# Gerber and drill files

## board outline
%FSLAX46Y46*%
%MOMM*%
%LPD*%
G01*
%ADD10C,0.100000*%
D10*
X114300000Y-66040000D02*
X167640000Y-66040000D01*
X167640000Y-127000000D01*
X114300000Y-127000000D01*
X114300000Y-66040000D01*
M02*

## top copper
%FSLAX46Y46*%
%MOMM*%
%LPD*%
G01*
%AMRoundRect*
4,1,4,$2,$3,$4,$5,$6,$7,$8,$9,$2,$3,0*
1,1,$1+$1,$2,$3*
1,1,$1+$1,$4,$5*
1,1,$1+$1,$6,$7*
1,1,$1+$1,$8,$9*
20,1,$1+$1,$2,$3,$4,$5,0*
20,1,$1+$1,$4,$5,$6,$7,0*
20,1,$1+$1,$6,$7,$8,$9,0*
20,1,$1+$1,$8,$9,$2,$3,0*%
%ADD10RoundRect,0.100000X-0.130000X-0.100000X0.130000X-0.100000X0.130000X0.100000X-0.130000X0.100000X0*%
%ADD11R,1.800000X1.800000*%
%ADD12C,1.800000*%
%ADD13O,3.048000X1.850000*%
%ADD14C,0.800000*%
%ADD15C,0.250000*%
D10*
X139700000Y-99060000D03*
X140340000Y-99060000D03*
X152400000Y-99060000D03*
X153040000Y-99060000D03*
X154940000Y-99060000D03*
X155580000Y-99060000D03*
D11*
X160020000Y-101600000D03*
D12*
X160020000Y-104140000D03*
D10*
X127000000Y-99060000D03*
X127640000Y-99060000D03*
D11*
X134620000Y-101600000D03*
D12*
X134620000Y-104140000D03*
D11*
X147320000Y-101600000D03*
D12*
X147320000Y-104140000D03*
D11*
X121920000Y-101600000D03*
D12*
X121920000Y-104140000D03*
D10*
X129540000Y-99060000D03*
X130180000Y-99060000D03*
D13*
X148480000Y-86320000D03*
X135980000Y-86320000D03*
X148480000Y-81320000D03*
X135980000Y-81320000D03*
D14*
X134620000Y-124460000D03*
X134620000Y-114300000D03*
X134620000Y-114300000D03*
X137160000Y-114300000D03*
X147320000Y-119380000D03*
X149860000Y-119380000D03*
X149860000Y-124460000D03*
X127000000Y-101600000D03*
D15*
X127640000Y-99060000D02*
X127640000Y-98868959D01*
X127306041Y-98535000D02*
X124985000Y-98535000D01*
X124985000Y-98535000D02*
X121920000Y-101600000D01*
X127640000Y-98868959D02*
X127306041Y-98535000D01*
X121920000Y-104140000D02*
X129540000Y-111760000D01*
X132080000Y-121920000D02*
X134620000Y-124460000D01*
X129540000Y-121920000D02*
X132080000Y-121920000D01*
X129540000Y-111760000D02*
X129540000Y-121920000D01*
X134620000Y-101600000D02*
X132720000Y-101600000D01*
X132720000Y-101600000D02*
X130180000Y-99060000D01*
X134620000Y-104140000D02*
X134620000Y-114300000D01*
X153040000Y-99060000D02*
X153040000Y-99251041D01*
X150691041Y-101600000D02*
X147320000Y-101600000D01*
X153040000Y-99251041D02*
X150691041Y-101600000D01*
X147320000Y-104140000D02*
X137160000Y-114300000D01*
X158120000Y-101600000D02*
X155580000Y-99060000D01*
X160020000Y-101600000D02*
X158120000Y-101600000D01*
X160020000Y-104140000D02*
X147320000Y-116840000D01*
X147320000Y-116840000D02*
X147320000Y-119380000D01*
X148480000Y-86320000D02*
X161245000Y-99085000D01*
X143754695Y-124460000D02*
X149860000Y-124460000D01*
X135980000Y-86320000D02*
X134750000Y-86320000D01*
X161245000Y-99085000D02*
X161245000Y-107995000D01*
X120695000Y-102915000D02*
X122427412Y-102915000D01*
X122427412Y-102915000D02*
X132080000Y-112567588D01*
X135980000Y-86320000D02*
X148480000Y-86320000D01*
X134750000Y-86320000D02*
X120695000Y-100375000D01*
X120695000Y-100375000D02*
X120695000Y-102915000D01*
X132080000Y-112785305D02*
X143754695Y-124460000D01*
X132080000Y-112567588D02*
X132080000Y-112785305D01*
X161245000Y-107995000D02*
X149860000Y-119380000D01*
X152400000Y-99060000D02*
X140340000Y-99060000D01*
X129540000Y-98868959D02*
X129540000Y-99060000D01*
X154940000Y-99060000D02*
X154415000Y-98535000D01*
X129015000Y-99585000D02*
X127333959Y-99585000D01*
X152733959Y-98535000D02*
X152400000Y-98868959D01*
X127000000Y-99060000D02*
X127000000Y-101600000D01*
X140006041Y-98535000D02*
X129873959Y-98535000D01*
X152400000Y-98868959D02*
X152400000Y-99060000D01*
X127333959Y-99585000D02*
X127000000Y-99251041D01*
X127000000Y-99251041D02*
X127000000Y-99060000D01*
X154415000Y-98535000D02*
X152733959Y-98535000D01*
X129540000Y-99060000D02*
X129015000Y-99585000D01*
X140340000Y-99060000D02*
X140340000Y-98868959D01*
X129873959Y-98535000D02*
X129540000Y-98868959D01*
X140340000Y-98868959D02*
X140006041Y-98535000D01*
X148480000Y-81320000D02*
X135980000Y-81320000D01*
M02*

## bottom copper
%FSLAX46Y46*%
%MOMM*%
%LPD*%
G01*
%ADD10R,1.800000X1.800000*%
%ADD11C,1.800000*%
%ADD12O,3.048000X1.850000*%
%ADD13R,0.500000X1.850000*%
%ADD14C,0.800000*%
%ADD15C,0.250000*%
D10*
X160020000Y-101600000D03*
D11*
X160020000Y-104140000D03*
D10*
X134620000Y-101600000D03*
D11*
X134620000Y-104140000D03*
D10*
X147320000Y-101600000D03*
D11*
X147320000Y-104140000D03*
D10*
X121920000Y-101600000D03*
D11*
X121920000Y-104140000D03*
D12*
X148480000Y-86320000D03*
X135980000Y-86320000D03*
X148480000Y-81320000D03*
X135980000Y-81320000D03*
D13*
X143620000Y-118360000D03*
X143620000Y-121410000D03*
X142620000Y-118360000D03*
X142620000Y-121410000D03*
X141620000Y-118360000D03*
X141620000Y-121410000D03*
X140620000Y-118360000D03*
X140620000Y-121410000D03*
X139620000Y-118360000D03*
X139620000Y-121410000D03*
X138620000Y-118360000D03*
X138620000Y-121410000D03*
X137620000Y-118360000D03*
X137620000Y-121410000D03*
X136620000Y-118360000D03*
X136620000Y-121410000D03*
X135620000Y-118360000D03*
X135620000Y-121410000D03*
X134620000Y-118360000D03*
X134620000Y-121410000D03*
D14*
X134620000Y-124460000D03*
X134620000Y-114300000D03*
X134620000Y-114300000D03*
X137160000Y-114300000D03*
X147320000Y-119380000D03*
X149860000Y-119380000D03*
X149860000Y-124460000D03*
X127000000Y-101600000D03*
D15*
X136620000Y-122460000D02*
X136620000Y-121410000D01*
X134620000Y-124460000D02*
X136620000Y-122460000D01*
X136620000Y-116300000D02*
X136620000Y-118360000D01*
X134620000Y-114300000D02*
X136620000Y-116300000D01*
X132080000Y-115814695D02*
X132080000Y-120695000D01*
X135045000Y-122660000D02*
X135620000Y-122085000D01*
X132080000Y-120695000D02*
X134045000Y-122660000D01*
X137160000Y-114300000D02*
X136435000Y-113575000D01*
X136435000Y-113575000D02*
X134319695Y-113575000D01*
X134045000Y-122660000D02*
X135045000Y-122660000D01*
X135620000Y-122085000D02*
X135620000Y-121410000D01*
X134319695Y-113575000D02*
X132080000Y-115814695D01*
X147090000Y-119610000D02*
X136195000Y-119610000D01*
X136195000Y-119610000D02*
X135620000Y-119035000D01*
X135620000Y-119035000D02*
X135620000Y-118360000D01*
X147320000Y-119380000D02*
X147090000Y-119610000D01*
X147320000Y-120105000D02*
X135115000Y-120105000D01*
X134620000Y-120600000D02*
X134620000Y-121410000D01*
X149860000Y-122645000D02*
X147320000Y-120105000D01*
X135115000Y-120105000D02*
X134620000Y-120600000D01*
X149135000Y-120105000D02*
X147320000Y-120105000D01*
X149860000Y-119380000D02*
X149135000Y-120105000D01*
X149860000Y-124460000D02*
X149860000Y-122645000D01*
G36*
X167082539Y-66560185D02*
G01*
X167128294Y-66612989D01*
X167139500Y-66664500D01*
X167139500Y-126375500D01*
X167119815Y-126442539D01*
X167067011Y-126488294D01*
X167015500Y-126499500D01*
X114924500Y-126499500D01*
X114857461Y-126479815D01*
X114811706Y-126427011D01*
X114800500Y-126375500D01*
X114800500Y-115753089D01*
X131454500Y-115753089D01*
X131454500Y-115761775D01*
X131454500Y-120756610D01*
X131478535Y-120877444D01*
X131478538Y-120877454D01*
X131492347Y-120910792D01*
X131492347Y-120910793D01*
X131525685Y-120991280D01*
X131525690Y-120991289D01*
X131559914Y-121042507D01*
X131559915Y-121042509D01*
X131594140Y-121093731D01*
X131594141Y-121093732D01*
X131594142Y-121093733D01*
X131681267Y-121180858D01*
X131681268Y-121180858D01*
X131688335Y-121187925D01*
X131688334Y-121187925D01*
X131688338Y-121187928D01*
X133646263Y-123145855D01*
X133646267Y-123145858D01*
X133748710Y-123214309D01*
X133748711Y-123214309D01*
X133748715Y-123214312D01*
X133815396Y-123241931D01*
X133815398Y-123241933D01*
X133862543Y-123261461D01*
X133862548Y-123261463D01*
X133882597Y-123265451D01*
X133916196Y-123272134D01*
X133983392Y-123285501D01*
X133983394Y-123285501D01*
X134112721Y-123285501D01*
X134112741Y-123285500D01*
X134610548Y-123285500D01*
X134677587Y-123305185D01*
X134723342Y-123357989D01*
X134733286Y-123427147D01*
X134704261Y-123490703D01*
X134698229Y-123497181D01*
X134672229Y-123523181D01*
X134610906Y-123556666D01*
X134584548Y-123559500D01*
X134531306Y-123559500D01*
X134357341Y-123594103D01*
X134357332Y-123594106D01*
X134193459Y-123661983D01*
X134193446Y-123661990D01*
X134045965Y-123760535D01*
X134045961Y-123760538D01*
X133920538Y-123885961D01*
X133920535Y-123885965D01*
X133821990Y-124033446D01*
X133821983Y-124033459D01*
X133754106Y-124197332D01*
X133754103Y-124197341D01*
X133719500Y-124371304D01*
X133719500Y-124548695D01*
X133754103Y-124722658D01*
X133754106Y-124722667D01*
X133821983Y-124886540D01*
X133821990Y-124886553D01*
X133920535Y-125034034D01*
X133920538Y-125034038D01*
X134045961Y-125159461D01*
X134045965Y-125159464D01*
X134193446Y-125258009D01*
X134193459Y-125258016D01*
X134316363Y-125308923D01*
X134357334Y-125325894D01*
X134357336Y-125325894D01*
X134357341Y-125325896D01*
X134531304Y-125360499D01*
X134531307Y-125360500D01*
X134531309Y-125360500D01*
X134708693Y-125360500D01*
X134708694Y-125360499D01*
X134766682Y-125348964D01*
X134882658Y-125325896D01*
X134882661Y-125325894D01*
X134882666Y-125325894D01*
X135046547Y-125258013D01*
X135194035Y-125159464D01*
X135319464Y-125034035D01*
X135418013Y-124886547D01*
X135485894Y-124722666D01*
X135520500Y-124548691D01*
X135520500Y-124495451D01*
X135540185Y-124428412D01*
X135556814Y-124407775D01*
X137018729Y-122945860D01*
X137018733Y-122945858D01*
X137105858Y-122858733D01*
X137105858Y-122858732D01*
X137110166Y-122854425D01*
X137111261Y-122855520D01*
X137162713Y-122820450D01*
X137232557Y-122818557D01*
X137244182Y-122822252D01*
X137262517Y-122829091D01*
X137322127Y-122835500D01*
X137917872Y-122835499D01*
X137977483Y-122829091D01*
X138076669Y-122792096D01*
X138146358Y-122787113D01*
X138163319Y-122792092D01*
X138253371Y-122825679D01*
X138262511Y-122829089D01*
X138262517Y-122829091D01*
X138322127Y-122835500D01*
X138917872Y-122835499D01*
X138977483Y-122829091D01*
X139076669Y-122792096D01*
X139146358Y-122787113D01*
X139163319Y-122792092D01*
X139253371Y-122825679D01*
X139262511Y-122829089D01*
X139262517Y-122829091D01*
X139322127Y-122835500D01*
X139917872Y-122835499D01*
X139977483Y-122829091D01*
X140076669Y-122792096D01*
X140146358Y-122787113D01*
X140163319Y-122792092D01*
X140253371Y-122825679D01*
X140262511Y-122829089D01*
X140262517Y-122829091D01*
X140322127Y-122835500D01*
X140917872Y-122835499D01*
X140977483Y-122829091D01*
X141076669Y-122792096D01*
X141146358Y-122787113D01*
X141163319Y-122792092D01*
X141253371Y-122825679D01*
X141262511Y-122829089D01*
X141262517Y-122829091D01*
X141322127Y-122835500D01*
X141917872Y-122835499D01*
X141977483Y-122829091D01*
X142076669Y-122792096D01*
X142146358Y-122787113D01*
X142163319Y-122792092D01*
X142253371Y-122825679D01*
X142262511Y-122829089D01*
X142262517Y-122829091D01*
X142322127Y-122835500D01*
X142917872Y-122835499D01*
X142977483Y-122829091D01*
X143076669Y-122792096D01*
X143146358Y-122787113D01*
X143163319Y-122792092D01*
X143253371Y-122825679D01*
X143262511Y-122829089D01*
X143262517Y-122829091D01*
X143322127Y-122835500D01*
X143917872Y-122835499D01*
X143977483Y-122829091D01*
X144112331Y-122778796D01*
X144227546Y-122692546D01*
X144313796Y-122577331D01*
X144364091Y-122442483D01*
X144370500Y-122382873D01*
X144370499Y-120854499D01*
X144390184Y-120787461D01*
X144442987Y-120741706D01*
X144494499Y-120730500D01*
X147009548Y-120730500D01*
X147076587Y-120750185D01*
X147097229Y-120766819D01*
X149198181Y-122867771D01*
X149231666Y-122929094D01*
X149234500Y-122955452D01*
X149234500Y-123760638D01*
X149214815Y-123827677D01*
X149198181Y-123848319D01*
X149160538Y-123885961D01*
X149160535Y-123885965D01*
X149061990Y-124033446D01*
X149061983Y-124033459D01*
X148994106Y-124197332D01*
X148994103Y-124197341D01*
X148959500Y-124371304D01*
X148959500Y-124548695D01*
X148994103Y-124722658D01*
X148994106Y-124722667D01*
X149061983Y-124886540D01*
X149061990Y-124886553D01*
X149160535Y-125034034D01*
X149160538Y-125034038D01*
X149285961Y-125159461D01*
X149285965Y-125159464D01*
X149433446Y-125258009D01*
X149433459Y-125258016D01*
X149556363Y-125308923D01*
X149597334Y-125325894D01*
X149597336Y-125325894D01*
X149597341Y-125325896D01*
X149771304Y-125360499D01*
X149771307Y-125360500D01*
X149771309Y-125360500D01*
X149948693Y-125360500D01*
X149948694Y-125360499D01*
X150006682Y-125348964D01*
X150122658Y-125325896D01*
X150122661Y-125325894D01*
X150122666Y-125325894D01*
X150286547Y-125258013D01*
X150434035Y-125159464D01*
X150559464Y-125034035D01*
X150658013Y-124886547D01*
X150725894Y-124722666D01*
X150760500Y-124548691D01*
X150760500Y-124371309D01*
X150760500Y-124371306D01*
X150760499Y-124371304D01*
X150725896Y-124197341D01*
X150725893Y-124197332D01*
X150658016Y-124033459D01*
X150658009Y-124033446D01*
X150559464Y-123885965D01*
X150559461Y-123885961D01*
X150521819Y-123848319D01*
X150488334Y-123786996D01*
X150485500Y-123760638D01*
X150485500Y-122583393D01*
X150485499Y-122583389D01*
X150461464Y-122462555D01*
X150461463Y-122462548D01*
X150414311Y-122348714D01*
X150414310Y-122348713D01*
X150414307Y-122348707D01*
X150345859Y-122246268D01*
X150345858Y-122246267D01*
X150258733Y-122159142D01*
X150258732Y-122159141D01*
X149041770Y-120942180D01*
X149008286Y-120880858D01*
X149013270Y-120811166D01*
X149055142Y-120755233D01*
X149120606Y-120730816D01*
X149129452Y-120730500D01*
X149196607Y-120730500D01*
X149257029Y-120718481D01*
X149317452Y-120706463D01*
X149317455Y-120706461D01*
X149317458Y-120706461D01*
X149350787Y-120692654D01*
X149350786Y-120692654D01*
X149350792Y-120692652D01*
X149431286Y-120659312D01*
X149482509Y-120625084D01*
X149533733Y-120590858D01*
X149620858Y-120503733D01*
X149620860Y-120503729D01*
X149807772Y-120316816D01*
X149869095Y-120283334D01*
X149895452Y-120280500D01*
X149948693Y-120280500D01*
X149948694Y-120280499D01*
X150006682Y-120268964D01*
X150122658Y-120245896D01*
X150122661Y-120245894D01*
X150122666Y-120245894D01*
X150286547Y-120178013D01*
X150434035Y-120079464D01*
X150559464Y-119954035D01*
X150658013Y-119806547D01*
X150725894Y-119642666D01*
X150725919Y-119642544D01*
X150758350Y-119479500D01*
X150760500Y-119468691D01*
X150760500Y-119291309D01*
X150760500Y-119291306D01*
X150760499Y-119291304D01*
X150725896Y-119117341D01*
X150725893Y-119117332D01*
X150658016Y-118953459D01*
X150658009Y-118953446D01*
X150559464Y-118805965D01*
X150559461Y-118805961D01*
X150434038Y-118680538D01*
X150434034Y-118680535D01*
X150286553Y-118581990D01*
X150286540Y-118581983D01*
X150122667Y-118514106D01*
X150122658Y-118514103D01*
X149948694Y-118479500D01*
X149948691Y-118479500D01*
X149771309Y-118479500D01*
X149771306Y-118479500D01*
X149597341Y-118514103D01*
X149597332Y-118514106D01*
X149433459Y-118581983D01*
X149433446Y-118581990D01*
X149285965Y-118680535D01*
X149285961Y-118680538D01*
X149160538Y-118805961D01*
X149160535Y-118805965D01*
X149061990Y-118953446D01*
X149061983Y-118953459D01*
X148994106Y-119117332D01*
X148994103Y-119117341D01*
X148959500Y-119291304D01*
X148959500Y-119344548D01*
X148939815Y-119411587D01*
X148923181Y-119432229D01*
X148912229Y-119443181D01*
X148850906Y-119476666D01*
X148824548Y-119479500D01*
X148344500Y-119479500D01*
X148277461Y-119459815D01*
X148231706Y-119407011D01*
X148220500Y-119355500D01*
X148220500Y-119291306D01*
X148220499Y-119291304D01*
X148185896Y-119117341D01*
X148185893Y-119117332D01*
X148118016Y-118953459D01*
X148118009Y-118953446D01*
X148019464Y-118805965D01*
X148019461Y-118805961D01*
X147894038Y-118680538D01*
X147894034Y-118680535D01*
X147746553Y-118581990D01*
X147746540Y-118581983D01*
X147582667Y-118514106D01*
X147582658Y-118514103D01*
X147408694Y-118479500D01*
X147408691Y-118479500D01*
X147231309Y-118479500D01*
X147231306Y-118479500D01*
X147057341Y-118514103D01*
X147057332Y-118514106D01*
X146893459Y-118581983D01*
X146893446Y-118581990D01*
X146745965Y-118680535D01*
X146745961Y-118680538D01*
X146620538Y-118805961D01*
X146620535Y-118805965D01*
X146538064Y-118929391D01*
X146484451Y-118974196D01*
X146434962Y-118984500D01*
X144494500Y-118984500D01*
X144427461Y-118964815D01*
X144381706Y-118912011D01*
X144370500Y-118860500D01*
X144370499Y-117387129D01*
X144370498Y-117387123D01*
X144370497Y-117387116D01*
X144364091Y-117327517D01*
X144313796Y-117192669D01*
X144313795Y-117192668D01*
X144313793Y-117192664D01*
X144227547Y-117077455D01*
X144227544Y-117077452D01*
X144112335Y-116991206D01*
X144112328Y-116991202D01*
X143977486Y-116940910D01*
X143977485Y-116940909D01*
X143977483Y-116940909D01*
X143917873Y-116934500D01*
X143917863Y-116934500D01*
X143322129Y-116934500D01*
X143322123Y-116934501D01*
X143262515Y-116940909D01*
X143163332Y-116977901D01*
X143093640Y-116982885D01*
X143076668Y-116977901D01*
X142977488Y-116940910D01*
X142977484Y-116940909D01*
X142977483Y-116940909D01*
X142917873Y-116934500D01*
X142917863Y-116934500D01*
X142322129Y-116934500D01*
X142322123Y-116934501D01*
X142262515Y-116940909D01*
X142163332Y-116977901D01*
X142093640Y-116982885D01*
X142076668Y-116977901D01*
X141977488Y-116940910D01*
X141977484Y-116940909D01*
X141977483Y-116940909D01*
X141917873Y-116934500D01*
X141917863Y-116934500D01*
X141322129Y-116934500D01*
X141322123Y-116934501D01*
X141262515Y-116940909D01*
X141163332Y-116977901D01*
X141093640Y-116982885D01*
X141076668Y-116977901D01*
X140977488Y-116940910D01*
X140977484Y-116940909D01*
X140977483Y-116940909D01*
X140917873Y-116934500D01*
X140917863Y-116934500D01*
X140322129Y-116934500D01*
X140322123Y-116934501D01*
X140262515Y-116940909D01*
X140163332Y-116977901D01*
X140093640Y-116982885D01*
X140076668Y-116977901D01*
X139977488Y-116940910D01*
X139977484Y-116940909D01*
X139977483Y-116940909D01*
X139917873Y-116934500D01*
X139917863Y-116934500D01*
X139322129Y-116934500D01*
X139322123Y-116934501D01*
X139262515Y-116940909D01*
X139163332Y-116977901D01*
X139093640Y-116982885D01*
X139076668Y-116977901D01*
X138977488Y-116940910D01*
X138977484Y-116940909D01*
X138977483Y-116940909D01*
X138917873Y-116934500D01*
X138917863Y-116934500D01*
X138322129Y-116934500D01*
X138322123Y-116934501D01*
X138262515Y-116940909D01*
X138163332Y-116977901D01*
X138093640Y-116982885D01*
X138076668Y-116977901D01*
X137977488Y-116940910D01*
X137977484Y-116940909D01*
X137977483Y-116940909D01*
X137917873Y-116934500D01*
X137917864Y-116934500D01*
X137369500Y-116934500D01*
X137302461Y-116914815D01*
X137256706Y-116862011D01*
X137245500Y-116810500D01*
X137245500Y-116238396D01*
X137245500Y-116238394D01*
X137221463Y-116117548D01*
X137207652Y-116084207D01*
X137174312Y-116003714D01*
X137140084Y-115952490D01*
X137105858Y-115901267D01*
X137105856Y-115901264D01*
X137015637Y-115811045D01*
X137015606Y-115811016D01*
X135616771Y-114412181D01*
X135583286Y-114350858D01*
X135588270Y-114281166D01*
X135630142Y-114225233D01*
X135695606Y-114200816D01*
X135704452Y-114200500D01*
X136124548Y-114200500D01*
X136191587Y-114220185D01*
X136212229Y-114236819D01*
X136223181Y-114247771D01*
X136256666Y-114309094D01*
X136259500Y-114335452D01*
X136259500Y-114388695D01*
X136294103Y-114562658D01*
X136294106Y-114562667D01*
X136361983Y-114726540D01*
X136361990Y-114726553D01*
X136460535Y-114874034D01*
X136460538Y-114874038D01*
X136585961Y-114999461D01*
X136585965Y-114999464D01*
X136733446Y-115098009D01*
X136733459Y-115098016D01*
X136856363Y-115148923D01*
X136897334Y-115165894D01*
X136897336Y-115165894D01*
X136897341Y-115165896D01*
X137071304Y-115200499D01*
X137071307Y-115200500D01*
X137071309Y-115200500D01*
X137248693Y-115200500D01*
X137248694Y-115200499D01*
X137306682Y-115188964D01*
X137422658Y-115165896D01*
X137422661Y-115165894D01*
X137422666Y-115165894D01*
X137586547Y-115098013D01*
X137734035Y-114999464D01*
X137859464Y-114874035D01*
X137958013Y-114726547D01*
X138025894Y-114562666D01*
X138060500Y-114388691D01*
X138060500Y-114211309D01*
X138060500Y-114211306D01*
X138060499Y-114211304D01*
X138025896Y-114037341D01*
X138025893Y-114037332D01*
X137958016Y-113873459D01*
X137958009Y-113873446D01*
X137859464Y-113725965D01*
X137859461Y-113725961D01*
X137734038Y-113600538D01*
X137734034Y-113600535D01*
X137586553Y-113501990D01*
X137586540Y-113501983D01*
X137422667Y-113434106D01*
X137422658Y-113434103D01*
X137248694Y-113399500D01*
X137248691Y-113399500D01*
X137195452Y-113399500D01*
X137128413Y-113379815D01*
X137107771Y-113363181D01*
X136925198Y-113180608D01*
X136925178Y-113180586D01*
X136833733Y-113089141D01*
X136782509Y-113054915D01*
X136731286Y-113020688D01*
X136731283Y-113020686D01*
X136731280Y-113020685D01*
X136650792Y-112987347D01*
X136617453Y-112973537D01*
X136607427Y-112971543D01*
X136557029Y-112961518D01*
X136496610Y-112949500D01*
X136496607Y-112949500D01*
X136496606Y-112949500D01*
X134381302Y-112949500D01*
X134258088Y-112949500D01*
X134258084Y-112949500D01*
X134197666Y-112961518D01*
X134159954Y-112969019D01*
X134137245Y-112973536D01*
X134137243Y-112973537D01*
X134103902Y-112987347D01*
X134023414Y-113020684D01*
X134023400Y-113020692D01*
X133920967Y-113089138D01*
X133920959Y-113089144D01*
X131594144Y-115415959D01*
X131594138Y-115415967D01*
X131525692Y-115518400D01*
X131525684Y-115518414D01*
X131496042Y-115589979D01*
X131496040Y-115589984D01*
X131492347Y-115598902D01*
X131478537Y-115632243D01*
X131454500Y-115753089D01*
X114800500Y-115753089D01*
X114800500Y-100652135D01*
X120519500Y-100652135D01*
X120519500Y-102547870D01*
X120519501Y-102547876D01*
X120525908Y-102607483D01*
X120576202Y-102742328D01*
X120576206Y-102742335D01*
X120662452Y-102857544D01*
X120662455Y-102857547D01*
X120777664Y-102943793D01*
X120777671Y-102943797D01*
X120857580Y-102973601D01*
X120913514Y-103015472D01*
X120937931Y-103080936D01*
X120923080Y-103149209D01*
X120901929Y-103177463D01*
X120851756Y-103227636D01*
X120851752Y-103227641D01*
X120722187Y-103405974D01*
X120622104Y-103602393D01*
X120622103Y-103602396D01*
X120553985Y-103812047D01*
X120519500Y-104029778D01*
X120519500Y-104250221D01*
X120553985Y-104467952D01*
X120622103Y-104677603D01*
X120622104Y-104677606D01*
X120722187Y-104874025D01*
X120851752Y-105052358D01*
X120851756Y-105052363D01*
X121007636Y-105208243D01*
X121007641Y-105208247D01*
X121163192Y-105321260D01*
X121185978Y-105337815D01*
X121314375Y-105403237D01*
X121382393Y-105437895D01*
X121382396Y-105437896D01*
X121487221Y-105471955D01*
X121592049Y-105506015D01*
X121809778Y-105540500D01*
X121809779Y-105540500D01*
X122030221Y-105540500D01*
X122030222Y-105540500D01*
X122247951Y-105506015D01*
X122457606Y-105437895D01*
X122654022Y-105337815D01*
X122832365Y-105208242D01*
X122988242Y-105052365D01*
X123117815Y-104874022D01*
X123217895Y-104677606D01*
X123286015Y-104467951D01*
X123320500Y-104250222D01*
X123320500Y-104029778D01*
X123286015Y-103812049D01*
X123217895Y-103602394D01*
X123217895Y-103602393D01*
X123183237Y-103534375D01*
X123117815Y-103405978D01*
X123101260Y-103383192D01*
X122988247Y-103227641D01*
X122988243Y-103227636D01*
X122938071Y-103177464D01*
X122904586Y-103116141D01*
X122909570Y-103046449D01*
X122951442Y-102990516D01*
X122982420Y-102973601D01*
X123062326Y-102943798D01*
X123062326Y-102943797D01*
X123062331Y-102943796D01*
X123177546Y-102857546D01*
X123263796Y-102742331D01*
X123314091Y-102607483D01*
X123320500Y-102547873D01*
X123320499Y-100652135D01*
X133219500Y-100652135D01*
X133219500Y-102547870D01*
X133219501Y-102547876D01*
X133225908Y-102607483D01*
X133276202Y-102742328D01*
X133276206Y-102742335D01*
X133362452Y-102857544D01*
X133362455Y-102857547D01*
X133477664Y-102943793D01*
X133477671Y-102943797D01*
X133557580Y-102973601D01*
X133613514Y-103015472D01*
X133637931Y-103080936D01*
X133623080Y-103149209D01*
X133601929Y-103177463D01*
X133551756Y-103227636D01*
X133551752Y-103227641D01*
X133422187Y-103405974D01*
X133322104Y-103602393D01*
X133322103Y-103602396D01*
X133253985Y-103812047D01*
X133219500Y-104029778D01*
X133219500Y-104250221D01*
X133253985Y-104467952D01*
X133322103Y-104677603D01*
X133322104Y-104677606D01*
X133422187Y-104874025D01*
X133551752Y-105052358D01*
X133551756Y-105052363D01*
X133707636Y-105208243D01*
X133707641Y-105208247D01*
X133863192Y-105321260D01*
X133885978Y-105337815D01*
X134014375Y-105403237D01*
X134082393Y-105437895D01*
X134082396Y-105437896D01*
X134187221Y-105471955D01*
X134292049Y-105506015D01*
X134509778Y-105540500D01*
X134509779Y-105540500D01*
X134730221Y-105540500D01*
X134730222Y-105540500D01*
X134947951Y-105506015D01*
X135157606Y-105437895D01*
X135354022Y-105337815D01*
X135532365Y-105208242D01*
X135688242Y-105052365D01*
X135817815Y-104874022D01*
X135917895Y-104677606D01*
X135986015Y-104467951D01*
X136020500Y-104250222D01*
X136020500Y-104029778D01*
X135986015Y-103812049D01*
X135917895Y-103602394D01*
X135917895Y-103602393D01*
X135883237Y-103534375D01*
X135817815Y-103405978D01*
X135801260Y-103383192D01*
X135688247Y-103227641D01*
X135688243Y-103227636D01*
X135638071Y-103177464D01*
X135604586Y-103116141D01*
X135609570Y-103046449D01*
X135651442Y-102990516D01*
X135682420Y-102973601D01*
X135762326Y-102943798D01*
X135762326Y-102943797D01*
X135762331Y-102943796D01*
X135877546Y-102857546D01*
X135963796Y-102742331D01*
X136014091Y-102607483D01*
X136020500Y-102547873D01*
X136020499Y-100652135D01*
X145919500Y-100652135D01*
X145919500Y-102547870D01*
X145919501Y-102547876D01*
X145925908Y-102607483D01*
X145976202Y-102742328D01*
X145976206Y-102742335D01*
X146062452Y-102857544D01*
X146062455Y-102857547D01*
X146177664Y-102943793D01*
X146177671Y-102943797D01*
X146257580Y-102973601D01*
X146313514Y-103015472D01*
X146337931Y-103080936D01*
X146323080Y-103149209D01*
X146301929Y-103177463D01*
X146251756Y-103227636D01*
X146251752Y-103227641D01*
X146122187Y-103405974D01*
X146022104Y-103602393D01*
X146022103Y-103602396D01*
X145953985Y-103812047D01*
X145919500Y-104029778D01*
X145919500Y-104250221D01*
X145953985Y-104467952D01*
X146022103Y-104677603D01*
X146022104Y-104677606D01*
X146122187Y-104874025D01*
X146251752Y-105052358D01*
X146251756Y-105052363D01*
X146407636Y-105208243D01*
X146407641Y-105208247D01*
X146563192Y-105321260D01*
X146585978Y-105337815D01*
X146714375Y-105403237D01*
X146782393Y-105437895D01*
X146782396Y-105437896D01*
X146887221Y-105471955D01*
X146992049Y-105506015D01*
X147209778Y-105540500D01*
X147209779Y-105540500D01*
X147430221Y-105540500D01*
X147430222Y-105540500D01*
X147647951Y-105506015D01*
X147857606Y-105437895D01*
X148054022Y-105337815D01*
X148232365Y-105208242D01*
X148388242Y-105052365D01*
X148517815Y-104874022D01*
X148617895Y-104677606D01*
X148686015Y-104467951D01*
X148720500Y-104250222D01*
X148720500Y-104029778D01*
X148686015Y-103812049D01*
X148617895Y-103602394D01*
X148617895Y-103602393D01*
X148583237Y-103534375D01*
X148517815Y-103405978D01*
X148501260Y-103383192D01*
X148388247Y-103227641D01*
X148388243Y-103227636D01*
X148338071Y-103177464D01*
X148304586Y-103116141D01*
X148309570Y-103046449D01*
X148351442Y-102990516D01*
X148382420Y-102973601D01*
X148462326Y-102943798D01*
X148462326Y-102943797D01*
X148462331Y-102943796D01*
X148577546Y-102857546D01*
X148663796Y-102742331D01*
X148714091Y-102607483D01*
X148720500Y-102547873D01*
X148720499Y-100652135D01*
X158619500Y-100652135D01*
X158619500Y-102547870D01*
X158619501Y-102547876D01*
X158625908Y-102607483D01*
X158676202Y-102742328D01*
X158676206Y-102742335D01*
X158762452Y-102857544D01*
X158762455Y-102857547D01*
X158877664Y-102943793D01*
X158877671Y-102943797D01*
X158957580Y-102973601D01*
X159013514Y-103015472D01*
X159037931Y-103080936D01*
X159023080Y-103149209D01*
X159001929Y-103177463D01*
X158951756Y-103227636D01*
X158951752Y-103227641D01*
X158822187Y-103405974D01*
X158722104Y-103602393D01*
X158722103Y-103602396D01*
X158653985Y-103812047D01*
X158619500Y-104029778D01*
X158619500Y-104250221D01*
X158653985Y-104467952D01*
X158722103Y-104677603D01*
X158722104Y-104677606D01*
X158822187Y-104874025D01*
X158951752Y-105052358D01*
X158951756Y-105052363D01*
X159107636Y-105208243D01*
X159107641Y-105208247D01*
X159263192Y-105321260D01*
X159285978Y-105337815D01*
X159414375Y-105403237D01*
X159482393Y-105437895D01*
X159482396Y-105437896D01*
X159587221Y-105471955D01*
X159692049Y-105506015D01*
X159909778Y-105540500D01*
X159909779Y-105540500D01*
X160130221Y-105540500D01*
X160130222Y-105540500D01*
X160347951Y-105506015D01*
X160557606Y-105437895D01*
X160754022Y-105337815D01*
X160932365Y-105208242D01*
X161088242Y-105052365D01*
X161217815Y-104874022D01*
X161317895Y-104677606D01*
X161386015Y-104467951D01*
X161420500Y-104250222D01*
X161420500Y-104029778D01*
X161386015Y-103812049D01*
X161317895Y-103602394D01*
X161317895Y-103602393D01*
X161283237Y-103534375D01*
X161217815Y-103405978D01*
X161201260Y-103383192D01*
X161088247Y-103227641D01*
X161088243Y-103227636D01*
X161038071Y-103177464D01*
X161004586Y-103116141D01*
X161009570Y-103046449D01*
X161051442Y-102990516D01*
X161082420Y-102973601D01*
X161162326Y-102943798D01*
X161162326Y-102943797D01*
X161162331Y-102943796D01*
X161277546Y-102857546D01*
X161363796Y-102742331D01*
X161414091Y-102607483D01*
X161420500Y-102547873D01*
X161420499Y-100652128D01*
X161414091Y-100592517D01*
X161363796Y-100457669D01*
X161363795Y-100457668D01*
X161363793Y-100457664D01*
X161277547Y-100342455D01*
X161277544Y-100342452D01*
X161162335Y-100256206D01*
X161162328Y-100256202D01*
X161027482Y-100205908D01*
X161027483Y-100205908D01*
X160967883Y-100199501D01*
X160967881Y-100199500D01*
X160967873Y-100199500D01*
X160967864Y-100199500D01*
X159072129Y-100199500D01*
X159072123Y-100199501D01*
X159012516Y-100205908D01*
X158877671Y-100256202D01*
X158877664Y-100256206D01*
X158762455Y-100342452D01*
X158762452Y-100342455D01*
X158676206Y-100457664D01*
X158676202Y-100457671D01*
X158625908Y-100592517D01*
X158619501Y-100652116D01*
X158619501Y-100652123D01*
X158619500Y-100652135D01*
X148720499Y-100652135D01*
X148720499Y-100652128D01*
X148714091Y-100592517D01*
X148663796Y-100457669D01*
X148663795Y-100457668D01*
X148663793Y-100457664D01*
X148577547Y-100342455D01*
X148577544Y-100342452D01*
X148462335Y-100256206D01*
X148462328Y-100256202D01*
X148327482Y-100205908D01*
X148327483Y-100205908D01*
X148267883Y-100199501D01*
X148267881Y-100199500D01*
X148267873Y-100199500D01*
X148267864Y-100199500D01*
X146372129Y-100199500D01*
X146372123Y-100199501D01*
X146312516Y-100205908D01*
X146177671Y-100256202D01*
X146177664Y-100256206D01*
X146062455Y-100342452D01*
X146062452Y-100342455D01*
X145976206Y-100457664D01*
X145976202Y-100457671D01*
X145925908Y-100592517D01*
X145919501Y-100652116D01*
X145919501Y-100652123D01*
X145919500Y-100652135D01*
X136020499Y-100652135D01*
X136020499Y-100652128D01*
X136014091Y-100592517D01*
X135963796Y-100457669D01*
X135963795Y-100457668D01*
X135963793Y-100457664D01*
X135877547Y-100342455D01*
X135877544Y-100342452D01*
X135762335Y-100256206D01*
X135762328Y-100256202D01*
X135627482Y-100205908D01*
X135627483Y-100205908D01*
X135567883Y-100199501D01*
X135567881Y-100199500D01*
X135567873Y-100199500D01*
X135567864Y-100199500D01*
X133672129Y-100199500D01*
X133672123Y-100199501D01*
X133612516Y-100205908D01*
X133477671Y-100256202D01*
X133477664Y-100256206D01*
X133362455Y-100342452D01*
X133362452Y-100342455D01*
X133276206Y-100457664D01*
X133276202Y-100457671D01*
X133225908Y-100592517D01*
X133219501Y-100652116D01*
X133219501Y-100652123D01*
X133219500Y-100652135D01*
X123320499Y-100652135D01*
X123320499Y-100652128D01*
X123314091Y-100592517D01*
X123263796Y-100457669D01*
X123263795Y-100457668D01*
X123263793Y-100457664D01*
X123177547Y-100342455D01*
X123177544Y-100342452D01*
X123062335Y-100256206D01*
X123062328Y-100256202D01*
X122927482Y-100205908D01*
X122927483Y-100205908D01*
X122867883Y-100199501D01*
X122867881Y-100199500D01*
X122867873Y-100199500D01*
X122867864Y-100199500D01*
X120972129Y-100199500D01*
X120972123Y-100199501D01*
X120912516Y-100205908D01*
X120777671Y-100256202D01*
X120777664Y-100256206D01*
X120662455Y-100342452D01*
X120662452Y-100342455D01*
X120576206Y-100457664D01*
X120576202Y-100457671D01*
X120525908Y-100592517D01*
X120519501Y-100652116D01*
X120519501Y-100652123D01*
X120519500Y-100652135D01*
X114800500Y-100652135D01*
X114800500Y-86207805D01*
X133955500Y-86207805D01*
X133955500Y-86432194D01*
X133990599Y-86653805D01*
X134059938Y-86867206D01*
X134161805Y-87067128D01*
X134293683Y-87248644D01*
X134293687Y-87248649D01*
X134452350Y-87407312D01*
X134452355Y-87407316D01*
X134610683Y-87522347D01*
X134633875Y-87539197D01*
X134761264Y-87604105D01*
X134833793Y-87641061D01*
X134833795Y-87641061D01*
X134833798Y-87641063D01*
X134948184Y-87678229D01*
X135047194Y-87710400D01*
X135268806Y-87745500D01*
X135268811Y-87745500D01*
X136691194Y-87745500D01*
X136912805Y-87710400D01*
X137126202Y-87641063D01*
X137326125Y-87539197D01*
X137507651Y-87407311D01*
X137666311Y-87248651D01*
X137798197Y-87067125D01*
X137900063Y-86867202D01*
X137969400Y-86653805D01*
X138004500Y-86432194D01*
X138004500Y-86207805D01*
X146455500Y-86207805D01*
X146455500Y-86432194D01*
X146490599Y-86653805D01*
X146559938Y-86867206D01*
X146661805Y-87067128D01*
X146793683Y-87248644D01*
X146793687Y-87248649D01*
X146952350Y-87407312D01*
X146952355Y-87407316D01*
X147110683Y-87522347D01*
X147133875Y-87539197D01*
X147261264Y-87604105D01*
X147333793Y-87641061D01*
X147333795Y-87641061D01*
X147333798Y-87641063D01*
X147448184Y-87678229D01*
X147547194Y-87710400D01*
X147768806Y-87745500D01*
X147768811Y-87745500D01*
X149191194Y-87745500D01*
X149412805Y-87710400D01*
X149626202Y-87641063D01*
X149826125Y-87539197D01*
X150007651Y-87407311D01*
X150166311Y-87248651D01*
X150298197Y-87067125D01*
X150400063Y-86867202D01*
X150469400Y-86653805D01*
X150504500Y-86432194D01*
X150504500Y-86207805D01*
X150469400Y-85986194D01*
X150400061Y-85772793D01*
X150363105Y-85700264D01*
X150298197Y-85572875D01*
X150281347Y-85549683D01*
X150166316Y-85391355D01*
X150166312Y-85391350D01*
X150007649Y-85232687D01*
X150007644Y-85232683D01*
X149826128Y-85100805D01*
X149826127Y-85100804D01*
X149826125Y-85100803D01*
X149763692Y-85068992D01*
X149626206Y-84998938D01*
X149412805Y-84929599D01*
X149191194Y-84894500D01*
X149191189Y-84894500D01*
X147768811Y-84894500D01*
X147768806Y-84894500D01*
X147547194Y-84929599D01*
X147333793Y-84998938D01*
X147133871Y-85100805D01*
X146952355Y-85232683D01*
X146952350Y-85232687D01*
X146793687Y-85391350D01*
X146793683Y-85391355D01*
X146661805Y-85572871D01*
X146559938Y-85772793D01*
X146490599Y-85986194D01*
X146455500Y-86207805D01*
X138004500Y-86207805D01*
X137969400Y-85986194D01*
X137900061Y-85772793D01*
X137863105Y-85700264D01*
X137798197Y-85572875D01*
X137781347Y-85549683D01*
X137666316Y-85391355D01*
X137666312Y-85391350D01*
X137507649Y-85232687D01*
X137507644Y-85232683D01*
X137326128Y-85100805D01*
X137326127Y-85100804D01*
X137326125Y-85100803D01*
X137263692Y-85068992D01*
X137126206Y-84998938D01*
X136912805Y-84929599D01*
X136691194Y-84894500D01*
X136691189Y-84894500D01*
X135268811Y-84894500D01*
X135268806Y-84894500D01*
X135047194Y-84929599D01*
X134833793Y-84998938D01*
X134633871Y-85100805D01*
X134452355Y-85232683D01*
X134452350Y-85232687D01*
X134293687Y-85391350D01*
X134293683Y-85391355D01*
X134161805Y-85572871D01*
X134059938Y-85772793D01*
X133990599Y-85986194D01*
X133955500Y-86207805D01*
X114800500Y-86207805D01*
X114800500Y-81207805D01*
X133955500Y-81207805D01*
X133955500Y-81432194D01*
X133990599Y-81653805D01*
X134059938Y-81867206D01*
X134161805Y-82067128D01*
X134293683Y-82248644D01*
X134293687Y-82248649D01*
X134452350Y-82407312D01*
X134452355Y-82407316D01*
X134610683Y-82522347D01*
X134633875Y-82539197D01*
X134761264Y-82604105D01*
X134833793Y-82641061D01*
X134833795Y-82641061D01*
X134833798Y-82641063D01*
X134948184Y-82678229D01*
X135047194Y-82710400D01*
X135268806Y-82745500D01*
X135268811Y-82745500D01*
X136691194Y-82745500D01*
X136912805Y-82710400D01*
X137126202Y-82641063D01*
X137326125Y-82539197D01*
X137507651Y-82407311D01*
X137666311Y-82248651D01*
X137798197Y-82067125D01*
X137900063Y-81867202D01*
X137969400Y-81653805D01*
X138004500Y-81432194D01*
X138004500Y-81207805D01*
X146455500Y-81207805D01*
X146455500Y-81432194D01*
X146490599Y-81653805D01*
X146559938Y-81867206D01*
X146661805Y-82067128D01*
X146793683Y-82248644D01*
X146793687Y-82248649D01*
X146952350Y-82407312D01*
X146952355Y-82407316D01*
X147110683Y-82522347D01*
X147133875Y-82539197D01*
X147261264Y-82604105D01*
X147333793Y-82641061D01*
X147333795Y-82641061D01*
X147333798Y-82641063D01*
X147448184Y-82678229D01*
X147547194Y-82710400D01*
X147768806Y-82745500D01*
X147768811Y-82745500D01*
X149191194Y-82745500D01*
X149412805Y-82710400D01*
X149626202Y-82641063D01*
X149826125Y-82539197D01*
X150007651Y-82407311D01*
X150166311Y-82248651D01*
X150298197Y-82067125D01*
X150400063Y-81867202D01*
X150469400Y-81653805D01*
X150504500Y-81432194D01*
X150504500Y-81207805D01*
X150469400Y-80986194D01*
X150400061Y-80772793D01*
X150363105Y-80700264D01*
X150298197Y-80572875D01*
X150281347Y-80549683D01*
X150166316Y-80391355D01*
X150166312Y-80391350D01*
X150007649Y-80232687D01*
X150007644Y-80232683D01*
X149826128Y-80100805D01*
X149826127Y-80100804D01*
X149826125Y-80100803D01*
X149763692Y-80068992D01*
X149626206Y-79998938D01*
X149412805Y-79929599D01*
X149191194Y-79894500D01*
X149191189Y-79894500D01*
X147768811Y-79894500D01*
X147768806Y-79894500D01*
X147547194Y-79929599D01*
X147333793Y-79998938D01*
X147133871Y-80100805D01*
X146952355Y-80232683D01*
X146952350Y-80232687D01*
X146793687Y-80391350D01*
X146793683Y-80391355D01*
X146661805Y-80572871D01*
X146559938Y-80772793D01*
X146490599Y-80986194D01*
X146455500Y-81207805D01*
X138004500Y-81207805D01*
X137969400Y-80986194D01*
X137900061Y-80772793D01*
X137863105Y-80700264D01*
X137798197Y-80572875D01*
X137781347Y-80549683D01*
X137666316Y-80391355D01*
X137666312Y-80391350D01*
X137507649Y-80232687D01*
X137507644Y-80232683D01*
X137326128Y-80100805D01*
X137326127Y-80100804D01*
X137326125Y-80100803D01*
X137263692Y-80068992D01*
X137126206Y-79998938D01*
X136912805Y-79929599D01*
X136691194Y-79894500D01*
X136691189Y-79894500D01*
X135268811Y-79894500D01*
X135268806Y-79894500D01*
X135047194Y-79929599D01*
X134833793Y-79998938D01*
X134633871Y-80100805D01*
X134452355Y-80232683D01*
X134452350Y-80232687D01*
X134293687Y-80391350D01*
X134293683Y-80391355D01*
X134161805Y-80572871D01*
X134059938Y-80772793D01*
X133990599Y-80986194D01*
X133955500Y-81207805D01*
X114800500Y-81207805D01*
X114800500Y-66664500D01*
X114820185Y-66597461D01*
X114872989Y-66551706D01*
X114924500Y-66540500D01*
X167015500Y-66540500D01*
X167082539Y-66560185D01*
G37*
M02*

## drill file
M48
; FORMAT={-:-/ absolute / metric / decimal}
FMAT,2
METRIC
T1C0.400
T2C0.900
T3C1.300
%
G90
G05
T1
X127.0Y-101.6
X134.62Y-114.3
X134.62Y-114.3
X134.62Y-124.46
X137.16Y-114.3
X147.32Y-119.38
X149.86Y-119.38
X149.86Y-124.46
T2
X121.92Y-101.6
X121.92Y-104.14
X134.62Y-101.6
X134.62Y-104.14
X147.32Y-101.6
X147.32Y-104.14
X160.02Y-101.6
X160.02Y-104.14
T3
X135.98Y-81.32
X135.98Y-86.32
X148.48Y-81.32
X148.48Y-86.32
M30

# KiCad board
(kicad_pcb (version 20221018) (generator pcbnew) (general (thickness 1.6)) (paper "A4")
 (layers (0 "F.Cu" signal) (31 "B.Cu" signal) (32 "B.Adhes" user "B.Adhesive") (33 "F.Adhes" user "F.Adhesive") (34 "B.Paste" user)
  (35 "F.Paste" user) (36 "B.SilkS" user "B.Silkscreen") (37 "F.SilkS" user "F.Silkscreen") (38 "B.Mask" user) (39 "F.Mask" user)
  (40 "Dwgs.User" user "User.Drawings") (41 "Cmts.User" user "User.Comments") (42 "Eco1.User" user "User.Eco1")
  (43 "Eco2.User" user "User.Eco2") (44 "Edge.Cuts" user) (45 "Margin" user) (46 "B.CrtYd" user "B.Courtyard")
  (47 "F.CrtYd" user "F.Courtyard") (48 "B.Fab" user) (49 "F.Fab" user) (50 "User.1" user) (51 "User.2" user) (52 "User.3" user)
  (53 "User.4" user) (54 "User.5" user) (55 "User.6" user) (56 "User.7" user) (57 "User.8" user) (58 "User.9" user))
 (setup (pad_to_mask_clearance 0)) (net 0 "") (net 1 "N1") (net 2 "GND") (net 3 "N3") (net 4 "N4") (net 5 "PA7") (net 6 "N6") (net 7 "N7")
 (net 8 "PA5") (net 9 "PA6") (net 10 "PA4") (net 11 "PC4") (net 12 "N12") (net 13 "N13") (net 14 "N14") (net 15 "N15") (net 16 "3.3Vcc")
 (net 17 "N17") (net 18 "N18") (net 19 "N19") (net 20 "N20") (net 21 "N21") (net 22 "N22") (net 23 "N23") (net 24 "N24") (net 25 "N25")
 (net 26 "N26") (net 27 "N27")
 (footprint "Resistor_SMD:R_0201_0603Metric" (layer "F.Cu") (at 140.02 99.06)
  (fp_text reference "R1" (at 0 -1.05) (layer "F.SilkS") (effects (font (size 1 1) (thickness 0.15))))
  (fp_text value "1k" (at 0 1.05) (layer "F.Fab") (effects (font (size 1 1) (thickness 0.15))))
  (pad "" smd roundrect (at -0.345 0) (size 0.318 0.36) (layers "F.Paste") (roundrect_rratio 0.25))
  (pad "" smd roundrect (at 0.345 0) (size 0.318 0.36) (layers "F.Paste") (roundrect_rratio 0.25))
  (pad "1" smd roundrect (at -0.32 0) (size 0.46 0.4) (layers "F.Cu" "F.Mask") (roundrect_rratio 0.25) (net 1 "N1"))
  (pad "2" smd roundrect (at 0.32 0) (size 0.46 0.4) (layers "F.Cu" "F.Mask") (roundrect_rratio 0.25) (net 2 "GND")))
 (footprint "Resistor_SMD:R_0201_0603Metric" (layer "F.Cu") (at 152.72 99.06)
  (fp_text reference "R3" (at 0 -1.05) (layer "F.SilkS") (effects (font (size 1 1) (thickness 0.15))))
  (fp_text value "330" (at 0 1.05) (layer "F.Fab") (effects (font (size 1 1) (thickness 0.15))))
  (pad "" smd roundrect (at -0.345 0) (size 0.318 0.36) (layers "F.Paste") (roundrect_rratio 0.25))
  (pad "" smd roundrect (at 0.345 0) (size 0.318 0.36) (layers "F.Paste") (roundrect_rratio 0.25))
  (pad "1" smd roundrect (at -0.32 0) (size 0.46 0.4) (layers "F.Cu" "F.Mask") (roundrect_rratio 0.25) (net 2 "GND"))
  (pad "2" smd roundrect (at 0.32 0) (size 0.46 0.4) (layers "F.Cu" "F.Mask") (roundrect_rratio 0.25) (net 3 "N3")))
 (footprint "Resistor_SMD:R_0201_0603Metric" (layer "F.Cu") (at 155.26 99.06)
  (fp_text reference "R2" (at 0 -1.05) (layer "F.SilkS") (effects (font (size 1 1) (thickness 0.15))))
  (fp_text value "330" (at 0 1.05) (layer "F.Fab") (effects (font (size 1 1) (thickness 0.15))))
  (pad "" smd roundrect (at -0.345 0) (size 0.318 0.36) (layers "F.Paste") (roundrect_rratio 0.25))
  (pad "" smd roundrect (at 0.345 0) (size 0.318 0.36) (layers "F.Paste") (roundrect_rratio 0.25))
  (pad "1" smd roundrect (at -0.32 0) (size 0.46 0.4) (layers "F.Cu" "F.Mask") (roundrect_rratio 0.25) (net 2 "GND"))
  (pad "2" smd roundrect (at 0.32 0) (size 0.46 0.4) (layers "F.Cu" "F.Mask") (roundrect_rratio 0.25) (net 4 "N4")))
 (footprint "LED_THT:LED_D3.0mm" (layer "F.Cu") (at 160.02 101.6 -90)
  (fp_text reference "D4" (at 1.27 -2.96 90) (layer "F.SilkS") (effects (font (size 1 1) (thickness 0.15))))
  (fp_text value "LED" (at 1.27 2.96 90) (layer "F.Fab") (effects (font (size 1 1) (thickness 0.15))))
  (pad "1" thru_hole rect (at 0 0 270) (size 1.8 1.8) (drill 0.9) (layers "*.Cu" "*.Mask") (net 4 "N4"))
  (pad "2" thru_hole circle (at 2.54 0 270) (size 1.8 1.8) (drill 0.9) (layers "*.Cu" "*.Mask") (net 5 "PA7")))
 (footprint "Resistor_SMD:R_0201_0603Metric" (layer "F.Cu") (at 127.32 99.06)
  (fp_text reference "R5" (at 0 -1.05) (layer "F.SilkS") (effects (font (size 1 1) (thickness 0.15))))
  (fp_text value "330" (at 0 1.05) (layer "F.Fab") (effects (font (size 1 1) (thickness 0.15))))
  (pad "" smd roundrect (at -0.345 0) (size 0.318 0.36) (layers "F.Paste") (roundrect_rratio 0.25))
  (pad "" smd roundrect (at 0.345 0) (size 0.318 0.36) (layers "F.Paste") (roundrect_rratio 0.25))
  (pad "1" smd roundrect (at -0.32 0) (size 0.46 0.4) (layers "F.Cu" "F.Mask") (roundrect_rratio 0.25) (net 2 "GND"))
  (pad "2" smd roundrect (at 0.32 0) (size 0.46 0.4) (layers "F.Cu" "F.Mask") (roundrect_rratio 0.25) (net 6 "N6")))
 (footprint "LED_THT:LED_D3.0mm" (layer "F.Cu") (at 134.62 101.6 -90)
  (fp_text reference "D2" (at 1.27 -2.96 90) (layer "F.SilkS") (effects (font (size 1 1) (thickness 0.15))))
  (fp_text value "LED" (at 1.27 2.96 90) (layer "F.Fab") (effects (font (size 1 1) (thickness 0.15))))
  (pad "1" thru_hole rect (at 0 0 270) (size 1.8 1.8) (drill 0.9) (layers "*.Cu" "*.Mask") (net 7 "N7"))
  (pad "2" thru_hole circle (at 2.54 0 270) (size 1.8 1.8) (drill 0.9) (layers "*.Cu" "*.Mask") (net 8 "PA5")))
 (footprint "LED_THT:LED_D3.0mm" (layer "F.Cu") (at 147.32 101.6 -90)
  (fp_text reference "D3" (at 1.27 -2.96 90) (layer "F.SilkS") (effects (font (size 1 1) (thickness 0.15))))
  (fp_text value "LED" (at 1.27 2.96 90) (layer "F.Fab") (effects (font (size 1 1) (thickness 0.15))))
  (pad "1" thru_hole rect (at 0 0 270) (size 1.8 1.8) (drill 0.9) (layers "*.Cu" "*.Mask") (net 3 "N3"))
  (pad "2" thru_hole circle (at 2.54 0 270) (size 1.8 1.8) (drill 0.9) (layers "*.Cu" "*.Mask") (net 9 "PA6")))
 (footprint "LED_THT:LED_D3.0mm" (layer "F.Cu") (at 121.92 101.6 -90)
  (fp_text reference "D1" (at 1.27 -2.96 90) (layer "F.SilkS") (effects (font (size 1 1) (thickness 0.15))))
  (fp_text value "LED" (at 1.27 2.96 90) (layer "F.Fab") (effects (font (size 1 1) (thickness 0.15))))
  (pad "1" thru_hole rect (at 0 0 270) (size 1.8 1.8) (drill 0.9) (layers "*.Cu" "*.Mask") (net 6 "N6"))
  (pad "2" thru_hole circle (at 2.54 0 270) (size 1.8 1.8) (drill 0.9) (layers "*.Cu" "*.Mask") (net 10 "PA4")))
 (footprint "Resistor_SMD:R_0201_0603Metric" (layer "F.Cu") (at 129.86 99.06)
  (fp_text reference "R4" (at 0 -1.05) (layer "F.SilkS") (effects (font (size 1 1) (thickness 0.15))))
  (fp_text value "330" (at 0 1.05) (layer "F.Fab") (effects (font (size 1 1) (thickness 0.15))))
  (pad "" smd roundrect (at -0.345 0) (size 0.318 0.36) (layers "F.Paste") (roundrect_rratio 0.25))
  (pad "" smd roundrect (at 0.345 0) (size 0.318 0.36) (layers "F.Paste") (roundrect_rratio 0.25))
  (pad "1" smd roundrect (at -0.32 0) (size 0.46 0.4) (layers "F.Cu" "F.Mask") (roundrect_rratio 0.25) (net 2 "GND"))
  (pad "2" smd roundrect (at 0.32 0) (size 0.46 0.4) (layers "F.Cu" "F.Mask") (roundrect_rratio 0.25) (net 7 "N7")))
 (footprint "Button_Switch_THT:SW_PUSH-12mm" (layer "F.Cu") (at 148.48 86.32 180)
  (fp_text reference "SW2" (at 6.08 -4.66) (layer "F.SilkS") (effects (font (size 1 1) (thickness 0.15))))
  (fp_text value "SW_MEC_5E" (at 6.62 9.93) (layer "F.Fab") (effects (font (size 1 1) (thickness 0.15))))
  (pad "1" thru_hole oval (at 0 0 180) (size 3.048 1.85) (drill 1.3) (layers "*.Cu" "*.Mask") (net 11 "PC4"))
  (pad "1" thru_hole oval (at 12.5 0 180) (size 3.048 1.85) (drill 1.3) (layers "*.Cu" "*.Mask") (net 11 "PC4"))
  (pad "2" thru_hole oval (at 0 5 180) (size 3.048 1.85) (drill 1.3) (layers "*.Cu" "*.Mask") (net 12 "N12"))
  (pad "2" thru_hole oval (at 12.5 5 180) (size 3.048 1.85) (drill 1.3) (layers "*.Cu" "*.Mask") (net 12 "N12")))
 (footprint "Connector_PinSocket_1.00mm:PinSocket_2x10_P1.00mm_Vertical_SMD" (layer "B.Cu") (at 139.12 119.885 90)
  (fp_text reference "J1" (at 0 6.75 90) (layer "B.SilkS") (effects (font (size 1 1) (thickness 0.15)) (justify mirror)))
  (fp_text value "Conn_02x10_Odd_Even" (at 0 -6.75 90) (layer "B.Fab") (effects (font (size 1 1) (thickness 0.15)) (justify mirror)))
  (pad "1" smd rect (at 1.525 4.5 90) (size 1.85 0.5) (layers "B.Cu" "B.Paste" "B.Mask") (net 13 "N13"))
  (pad "2" smd rect (at -1.525 4.5 90) (size 1.85 0.5) (layers "B.Cu" "B.Paste" "B.Mask") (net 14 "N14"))
  (pad "3" smd rect (at 1.525 3.5 90) (size 1.85 0.5) (layers "B.Cu" "B.Paste" "B.Mask") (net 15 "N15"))
  (pad "4" smd rect (at -1.525 3.5 90) (size 1.85 0.5) (layers "B.Cu" "B.Paste" "B.Mask") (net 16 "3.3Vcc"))
  (pad "5" smd rect (at 1.525 2.5 90) (size 1.85 0.5) (layers "B.Cu" "B.Paste" "B.Mask") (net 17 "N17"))
  (pad "6" smd rect (at -1.525 2.5 90) (size 1.85 0.5) (layers "B.Cu" "B.Paste" "B.Mask") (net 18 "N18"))
  (pad "7" smd rect (at 1.525 1.5 90) (size 1.85 0.5) (layers "B.Cu" "B.Paste" "B.Mask") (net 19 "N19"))
  (pad "8" smd rect (at -1.525 1.5 90) (size 1.85 0.5) (layers "B.Cu" "B.Paste" "B.Mask") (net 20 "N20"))
  (pad "9" smd rect (at 1.525 0.5 90) (size 1.85 0.5) (layers "B.Cu" "B.Paste" "B.Mask") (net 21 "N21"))
  (pad "10" smd rect (at -1.525 0.5 90) (size 1.85 0.5) (layers "B.Cu" "B.Paste" "B.Mask") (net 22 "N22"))
  (pad "11" smd rect (at 1.525 -0.5 90) (size 1.85 0.5) (layers "B.Cu" "B.Paste" "B.Mask") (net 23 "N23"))
  (pad "12" smd rect (at -1.525 -0.5 90) (size 1.85 0.5) (layers "B.Cu" "B.Paste" "B.Mask") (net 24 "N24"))
  (pad "13" smd rect (at 1.525 -1.5 90) (size 1.85 0.5) (layers "B.Cu" "B.Paste" "B.Mask") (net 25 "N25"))
  (pad "14" smd rect (at -1.525 -1.5 90) (size 1.85 0.5) (layers "B.Cu" "B.Paste" "B.Mask") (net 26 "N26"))
  (pad "15" smd rect (at 1.525 -2.5 90) (size 1.85 0.5) (layers "B.Cu" "B.Paste" "B.Mask") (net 8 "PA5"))
  (pad "16" smd rect (at -1.525 -2.5 90) (size 1.85 0.5) (layers "B.Cu" "B.Paste" "B.Mask") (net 10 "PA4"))
  (pad "17" smd rect (at 1.525 -3.5 90) (size 1.85 0.5) (layers "B.Cu" "B.Paste" "B.Mask") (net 5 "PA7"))
  (pad "18" smd rect (at -1.525 -3.5 90) (size 1.85 0.5) (layers "B.Cu" "B.Paste" "B.Mask") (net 9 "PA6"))
  (pad "19" smd rect (at 1.525 -4.5 90) (size 1.85 0.5) (layers "B.Cu" "B.Paste" "B.Mask") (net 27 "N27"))
  (pad "20" smd rect (at -1.525 -4.5 90) (size 1.85 0.5) (layers "B.Cu" "B.Paste" "B.Mask") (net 11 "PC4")))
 (gr_rect (start 114.3 66.04) (end 167.64 127) (stroke (width 0.1) (type default)) (fill none) (layer "Edge.Cuts"))
 (segment (start 127.64 99.06) (end 127.64 98.868959) (width 0.25) (layer "F.Cu") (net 6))
 (segment (start 127.306041 98.535) (end 124.985 98.535) (width 0.25) (layer "F.Cu") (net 6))
 (segment (start 124.985 98.535) (end 121.92 101.6) (width 0.25) (layer "F.Cu") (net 6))
 (segment (start 127.64 98.868959) (end 127.306041 98.535) (width 0.25) (layer "F.Cu") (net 6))
 (segment (start 121.92 104.14) (end 129.54 111.76) (width 0.25) (layer "F.Cu") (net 10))
 (segment (start 132.08 121.92) (end 134.62 124.46) (width 0.25) (layer "F.Cu") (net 10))
 (segment (start 129.54 121.92) (end 132.08 121.92) (width 0.25) (layer "F.Cu") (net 10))
 (segment (start 129.54 111.76) (end 129.54 121.92) (width 0.25) (layer "F.Cu") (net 10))
 (via (at 134.62 124.46) (size 0.8) (drill 0.4) (layers "F.Cu" "B.Cu") (free) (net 10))
 (segment (start 136.62 122.46) (end 136.62 121.41) (width 0.25) (layer "B.Cu") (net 10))
 (segment (start 134.62 124.46) (end 136.62 122.46) (width 0.25) (layer "B.Cu") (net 10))
 (segment (start 134.62 101.6) (end 132.72 101.6) (width 0.25) (layer "F.Cu") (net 7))
 (segment (start 132.72 101.6) (end 130.18 99.06) (width 0.25) (layer "F.Cu") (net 7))
 (segment (start 134.62 104.14) (end 134.62 114.3) (width 0.25) (layer "F.Cu") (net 8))
 (via (at 134.62 114.3) (size 0.8) (drill 0.4) (layers "F.Cu" "B.Cu") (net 8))
 (via (at 134.62 114.3) (size 0.8) (drill 0.4) (layers "F.Cu" "B.Cu") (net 8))
 (segment (start 136.62 116.3) (end 136.62 118.36) (width 0.25) (layer "B.Cu") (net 8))
 (segment (start 134.62 114.3) (end 136.62 116.3) (width 0.25) (layer "B.Cu") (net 8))
 (segment (start 153.04 99.06) (end 153.04 99.251041) (width 0.25) (layer "F.Cu") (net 3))
 (segment (start 150.691041 101.6) (end 147.32 101.6) (width 0.25) (layer "F.Cu") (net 3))
 (segment (start 153.04 99.251041) (end 150.691041 101.6) (width 0.25) (layer "F.Cu") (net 3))
 (segment (start 147.32 104.14) (end 137.16 114.3) (width 0.25) (layer "F.Cu") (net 9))
 (via (at 137.16 114.3) (size 0.8) (drill 0.4) (layers "F.Cu" "B.Cu") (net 9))
 (segment (start 132.08 115.814695) (end 132.08 120.695) (width 0.25) (layer "B.Cu") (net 9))
 (segment (start 135.045 122.66) (end 135.62 122.085) (width 0.25) (layer "B.Cu") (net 9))
 (segment (start 132.08 120.695) (end 134.045 122.66) (width 0.25) (layer "B.Cu") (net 9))
 (segment (start 137.16 114.3) (end 136.435 113.575) (width 0.25) (layer "B.Cu") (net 9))
 (segment (start 136.435 113.575) (end 134.319695 113.575) (width 0.25) (layer "B.Cu") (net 9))
 (segment (start 134.045 122.66) (end 135.045 122.66) (width 0.25) (layer "B.Cu") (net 9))
 (segment (start 135.62 122.085) (end 135.62 121.41) (width 0.25) (layer "B.Cu") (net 9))
 (segment (start 134.319695 113.575) (end 132.08 115.814695) (width 0.25) (layer "B.Cu") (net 9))
 (segment (start 158.12 101.6) (end 155.58 99.06) (width 0.25) (layer "F.Cu") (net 4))
 (segment (start 160.02 101.6) (end 158.12 101.6) (width 0.25) (layer "F.Cu") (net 4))
 (segment (start 160.02 104.14) (end 147.32 116.84) (width 0.25) (layer "F.Cu") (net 5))
 (segment (start 147.32 116.84) (end 147.32 119.38) (width 0.25) (layer "F.Cu") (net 5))
 (via (at 147.32 119.38) (size 0.8) (drill 0.4) (layers "F.Cu" "B.Cu") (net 5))
 (segment (start 147.09 119.61) (end 136.195 119.61) (width 0.25) (layer "B.Cu") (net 5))
 (segment (start 136.195 119.61) (end 135.62 119.035) (width 0.25) (layer "B.Cu") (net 5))
 (segment (start 135.62 119.035) (end 135.62 118.36) (width 0.25) (layer "B.Cu") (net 5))
 (segment (start 147.32 119.38) (end 147.09 119.61) (width 0.25) (layer "B.Cu") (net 5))
 (segment (start 148.48 86.32) (end 161.245 99.085) (width 0.25) (layer "F.Cu") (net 11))
 (segment (start 143.754695 124.46) (end 149.86 124.46) (width 0.25) (layer "F.Cu") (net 11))
 (segment (start 135.98 86.32) (end 134.75 86.32) (width 0.25) (layer "F.Cu") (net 11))
 (segment (start 161.245 99.085) (end 161.245 107.995) (width 0.25) (layer "F.Cu") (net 11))
 (segment (start 120.695 102.915) (end 122.427412 102.915) (width 0.25) (layer "F.Cu") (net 11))
 (segment (start 122.427412 102.915) (end 132.08 112.567588) (width 0.25) (layer "F.Cu") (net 11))
 (segment (start 135.98 86.32) (end 148.48 86.32) (width 0.25) (layer "F.Cu") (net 11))
 (segment (start 134.75 86.32) (end 120.695 100.375) (width 0.25) (layer "F.Cu") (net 11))
 (segment (start 120.695 100.375) (end 120.695 102.915) (width 0.25) (layer "F.Cu") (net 11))
 (segment (start 132.08 112.785305) (end 143.754695 124.46) (width 0.25) (layer "F.Cu") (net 11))
 (segment (start 132.08 112.567588) (end 132.08 112.785305) (width 0.25) (layer "F.Cu") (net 11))
 (segment (start 161.245 107.995) (end 149.86 119.38) (width 0.25) (layer "F.Cu") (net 11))
 (via (at 149.86 119.38) (size 0.8) (drill 0.4) (layers "F.Cu" "B.Cu") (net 11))
 (via (at 149.86 124.46) (size 0.8) (drill 0.4) (layers "F.Cu" "B.Cu") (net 11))
 (segment (start 147.32 120.105) (end 135.115 120.105) (width 0.25) (layer "B.Cu") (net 11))
 (segment (start 134.62 120.6) (end 134.62 121.41) (width 0.25) (layer "B.Cu") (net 11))
 (segment (start 149.86 122.645) (end 147.32 120.105) (width 0.25) (layer "B.Cu") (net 11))
 (segment (start 135.115 120.105) (end 134.62 120.6) (width 0.25) (layer "B.Cu") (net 11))
 (segment (start 149.135 120.105) (end 147.32 120.105) (width 0.25) (layer "B.Cu") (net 11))
 (segment (start 149.86 119.38) (end 149.135 120.105) (width 0.25) (layer "B.Cu") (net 11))
 (segment (start 149.86 124.46) (end 149.86 122.645) (width 0.25) (layer "B.Cu") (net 11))
 (segment (start 152.4 99.06) (end 140.34 99.06) (width 0.25) (layer "F.Cu") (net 2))
 (segment (start 129.54 98.868959) (end 129.54 99.06) (width 0.25) (layer "F.Cu") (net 2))
 (segment (start 154.94 99.06) (end 154.415 98.535) (width 0.25) (layer "F.Cu") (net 2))
 (segment (start 129.015 99.585) (end 127.333959 99.585) (width 0.25) (layer "F.Cu") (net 2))
 (segment (start 152.733959 98.535) (end 152.4 98.868959) (width 0.25) (layer "F.Cu") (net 2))
 (segment (start 127 99.06) (end 127 101.6) (width 0.25) (layer "F.Cu") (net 2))
 (segment (start 140.006041 98.535) (end 129.873959 98.535) (width 0.25) (layer "F.Cu") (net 2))
 (segment (start 152.4 98.868959) (end 152.4 99.06) (width 0.25) (layer "F.Cu") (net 2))
 (segment (start 127.333959 99.585) (end 127 99.251041) (width 0.25) (layer "F.Cu") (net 2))
 (segment (start 127 99.251041) (end 127 99.06) (width 0.25) (layer "F.Cu") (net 2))
 (segment (start 154.415 98.535) (end 152.733959 98.535) (width 0.25) (layer "F.Cu") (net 2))
 (segment (start 129.54 99.06) (end 129.015 99.585) (width 0.25) (layer "F.Cu") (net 2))
 (segment (start 140.34 99.06) (end 140.34 98.868959) (width 0.25) (layer "F.Cu") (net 2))
 (segment (start 129.873959 98.535) (end 129.54 98.868959) (width 0.25) (layer "F.Cu") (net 2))
 (segment (start 140.34 98.868959) (end 140.006041 98.535) (width 0.25) (layer "F.Cu") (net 2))
 (via (at 127 101.6) (size 0.8) (drill 0.4) (layers "F.Cu" "B.Cu") (free) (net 2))
 (segment (start 148.48 81.32) (end 135.98 81.32) (width 0.25) (layer "F.Cu") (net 12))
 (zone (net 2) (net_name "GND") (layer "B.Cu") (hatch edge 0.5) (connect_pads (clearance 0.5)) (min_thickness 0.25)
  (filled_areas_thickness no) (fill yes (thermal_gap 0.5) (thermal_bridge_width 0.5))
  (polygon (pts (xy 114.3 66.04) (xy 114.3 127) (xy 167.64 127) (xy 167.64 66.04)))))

